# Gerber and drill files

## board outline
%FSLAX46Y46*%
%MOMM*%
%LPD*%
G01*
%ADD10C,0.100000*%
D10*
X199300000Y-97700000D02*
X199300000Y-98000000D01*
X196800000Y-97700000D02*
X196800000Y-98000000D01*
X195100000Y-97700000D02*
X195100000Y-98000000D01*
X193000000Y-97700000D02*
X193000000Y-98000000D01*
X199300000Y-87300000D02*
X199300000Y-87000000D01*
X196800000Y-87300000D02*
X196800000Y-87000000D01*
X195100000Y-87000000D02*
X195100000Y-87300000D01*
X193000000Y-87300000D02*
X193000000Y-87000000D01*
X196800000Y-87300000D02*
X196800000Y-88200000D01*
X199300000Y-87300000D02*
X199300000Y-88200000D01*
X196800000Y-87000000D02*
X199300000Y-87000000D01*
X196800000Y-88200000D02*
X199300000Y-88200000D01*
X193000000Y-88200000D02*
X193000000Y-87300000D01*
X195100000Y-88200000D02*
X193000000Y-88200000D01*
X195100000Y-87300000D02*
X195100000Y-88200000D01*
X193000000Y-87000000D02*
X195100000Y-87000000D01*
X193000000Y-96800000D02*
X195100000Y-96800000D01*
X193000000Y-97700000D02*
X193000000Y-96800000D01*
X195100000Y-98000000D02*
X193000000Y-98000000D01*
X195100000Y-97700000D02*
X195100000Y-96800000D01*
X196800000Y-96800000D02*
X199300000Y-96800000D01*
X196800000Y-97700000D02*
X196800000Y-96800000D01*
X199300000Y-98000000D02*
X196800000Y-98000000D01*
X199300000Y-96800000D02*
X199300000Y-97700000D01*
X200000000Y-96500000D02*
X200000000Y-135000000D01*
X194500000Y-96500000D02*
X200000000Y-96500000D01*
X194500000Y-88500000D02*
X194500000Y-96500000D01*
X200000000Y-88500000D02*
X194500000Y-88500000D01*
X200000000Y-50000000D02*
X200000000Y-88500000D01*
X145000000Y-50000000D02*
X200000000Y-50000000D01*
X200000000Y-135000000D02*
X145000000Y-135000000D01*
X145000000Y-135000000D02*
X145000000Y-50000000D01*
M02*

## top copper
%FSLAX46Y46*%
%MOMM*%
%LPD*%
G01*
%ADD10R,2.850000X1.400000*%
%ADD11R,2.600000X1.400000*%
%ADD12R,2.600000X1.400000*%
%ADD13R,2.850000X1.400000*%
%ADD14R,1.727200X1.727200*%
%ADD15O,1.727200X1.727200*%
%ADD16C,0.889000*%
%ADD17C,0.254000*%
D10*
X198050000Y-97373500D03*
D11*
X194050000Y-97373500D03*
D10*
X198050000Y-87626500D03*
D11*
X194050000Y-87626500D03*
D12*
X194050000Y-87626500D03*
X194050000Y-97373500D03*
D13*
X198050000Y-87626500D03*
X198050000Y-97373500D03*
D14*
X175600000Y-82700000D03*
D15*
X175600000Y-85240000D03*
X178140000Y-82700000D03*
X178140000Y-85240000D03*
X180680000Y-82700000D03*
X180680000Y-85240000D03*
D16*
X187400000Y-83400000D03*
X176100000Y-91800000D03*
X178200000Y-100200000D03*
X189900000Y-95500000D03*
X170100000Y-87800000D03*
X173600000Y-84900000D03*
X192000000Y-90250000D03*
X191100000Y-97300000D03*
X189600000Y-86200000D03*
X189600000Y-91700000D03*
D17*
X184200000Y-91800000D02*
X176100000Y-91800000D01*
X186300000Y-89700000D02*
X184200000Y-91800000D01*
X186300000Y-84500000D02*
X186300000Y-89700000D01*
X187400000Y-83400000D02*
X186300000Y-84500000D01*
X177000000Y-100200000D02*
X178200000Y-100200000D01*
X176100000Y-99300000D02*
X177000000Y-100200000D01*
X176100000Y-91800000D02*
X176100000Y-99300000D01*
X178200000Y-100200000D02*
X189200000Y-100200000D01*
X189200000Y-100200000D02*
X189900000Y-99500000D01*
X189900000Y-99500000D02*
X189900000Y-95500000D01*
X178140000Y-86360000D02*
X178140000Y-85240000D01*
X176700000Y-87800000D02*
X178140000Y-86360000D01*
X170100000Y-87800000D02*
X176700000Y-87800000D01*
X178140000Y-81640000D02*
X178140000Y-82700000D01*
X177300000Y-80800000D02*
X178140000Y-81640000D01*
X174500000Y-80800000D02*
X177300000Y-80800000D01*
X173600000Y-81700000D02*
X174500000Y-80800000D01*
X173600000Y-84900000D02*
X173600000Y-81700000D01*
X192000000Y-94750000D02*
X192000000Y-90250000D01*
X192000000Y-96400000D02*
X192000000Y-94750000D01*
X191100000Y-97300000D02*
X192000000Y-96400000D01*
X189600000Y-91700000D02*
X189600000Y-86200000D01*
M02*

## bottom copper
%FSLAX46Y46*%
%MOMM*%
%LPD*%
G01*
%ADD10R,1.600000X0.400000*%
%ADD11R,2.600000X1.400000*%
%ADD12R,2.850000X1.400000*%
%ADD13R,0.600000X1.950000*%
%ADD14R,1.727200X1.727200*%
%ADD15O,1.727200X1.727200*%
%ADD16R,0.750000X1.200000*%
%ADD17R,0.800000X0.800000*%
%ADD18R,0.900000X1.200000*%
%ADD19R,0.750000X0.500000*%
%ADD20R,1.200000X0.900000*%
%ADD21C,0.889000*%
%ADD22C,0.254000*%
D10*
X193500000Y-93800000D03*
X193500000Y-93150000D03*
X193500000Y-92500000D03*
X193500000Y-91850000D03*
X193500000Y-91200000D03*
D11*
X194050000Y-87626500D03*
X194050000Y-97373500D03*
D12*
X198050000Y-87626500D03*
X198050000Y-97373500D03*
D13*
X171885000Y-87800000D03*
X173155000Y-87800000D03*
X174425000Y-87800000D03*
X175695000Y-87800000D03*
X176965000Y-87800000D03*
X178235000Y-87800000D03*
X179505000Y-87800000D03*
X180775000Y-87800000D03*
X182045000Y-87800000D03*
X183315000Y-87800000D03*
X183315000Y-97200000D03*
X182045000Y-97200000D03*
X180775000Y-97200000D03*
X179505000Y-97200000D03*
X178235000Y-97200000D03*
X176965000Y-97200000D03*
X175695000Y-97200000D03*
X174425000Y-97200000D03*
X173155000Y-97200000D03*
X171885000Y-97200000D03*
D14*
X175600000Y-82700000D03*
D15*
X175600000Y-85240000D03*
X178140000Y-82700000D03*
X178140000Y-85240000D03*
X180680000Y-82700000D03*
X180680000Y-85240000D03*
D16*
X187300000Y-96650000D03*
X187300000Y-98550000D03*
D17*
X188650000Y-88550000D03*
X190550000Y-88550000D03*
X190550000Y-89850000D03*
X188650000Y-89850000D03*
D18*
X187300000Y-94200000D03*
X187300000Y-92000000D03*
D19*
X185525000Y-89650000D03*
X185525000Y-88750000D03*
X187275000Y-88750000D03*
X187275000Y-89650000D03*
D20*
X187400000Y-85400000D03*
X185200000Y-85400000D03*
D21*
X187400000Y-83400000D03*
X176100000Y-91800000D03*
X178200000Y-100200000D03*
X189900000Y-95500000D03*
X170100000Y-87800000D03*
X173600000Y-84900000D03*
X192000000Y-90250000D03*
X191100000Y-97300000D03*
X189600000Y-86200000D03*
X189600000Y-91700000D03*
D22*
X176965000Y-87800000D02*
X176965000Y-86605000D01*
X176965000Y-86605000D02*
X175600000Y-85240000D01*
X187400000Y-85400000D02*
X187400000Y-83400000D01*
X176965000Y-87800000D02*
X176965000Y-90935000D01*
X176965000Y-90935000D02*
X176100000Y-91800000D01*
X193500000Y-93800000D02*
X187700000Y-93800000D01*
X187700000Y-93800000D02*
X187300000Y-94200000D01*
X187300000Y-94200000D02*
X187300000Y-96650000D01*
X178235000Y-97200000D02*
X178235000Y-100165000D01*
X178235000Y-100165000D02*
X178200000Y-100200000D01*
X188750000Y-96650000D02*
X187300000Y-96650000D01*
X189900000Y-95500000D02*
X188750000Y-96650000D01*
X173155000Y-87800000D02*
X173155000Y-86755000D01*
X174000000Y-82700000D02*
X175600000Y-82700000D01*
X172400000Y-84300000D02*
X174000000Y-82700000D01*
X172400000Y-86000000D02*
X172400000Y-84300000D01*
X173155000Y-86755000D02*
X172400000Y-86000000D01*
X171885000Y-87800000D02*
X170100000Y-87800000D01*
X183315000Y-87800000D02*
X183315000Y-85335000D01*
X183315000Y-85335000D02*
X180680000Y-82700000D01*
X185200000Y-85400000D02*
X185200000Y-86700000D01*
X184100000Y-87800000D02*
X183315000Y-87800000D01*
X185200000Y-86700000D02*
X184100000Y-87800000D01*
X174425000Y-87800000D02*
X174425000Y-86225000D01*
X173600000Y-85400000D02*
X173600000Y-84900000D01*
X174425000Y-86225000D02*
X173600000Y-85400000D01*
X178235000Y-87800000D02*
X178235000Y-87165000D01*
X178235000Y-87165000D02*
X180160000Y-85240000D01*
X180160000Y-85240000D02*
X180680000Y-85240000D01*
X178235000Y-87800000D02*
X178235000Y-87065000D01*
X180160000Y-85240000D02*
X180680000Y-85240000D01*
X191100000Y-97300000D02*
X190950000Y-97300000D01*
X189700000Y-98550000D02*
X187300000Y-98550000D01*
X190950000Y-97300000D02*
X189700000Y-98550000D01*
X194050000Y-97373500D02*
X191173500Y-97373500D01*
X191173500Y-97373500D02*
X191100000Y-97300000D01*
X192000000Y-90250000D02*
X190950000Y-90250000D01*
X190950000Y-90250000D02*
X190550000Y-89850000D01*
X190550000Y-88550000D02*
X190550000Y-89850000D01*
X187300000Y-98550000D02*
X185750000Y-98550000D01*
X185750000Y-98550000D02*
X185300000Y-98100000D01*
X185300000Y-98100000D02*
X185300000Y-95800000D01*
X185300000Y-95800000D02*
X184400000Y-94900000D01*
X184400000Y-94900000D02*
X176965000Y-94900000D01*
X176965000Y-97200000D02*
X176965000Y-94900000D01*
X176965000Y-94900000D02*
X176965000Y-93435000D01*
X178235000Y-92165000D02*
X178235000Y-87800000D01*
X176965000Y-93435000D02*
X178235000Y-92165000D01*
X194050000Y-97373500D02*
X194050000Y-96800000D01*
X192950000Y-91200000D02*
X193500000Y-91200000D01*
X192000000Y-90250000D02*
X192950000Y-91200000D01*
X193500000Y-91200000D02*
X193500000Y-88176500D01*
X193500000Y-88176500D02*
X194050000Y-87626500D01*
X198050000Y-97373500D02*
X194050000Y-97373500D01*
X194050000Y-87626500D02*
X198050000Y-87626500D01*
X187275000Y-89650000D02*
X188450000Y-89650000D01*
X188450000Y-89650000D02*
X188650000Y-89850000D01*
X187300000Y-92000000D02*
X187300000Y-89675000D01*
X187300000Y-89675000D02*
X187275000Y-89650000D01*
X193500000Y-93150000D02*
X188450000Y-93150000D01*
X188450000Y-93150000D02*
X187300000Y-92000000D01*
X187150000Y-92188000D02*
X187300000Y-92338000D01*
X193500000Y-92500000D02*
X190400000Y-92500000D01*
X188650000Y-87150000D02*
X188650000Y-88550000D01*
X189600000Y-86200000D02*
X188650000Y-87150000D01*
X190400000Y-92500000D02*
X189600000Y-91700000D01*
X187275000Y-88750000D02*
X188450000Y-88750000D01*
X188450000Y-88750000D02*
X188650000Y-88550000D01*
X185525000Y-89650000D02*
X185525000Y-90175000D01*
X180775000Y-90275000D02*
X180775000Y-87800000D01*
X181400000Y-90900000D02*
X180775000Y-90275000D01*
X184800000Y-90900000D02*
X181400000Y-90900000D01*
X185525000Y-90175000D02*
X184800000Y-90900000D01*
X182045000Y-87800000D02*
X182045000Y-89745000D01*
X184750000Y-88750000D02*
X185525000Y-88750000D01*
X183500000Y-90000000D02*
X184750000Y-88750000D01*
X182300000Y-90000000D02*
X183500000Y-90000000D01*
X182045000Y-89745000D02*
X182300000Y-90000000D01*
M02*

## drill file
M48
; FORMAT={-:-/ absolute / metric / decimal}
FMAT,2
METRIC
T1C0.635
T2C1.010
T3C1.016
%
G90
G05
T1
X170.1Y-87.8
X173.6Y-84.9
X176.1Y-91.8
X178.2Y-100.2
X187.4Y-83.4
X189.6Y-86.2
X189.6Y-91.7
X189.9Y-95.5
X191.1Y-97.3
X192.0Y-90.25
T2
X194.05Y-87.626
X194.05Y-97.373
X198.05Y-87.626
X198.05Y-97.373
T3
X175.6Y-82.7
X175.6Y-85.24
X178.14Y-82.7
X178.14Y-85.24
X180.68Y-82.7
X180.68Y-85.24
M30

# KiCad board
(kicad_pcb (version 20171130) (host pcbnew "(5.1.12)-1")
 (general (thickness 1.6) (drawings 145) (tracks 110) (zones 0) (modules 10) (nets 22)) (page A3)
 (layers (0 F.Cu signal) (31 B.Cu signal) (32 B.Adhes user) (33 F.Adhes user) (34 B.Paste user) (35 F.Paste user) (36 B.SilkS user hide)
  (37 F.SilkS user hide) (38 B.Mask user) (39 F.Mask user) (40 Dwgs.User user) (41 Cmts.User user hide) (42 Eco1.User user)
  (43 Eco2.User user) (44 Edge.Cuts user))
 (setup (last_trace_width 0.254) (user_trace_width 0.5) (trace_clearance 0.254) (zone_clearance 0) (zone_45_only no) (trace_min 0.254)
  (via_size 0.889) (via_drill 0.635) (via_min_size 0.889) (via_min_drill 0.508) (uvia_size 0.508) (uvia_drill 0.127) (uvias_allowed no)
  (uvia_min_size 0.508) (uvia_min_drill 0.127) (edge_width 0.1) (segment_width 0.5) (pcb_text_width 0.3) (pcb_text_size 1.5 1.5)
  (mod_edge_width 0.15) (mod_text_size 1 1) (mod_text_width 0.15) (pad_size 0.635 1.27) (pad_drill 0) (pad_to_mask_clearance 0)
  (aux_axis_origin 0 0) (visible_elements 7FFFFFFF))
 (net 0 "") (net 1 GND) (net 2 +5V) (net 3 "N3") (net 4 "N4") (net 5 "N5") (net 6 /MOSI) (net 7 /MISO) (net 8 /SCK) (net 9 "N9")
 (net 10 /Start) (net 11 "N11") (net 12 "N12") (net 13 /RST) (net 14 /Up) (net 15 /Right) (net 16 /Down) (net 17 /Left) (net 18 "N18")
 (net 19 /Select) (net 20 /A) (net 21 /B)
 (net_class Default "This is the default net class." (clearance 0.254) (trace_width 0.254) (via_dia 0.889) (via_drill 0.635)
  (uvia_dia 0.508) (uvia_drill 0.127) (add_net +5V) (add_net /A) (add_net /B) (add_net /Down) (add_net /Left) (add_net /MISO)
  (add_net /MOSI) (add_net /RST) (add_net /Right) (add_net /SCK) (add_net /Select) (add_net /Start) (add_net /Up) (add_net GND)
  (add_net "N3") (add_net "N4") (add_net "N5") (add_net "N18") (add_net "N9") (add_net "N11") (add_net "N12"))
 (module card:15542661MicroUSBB (layer B.Cu) (at 194.5 92.5 270)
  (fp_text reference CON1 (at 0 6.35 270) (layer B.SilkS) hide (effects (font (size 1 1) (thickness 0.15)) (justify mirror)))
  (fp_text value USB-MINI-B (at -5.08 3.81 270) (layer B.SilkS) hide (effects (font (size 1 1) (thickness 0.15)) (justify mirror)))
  (pad 9 smd rect (at 4.8735 -3.55 270) (size 1.4 2.85) (layers F.Cu B.Paste B.Mask) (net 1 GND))
  (pad 7 smd rect (at 4.8735 0.45 270) (size 1.4 2.6) (layers F.Cu B.Paste B.Mask) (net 1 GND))
  (pad 8 smd rect (at -4.8735 -3.55 270) (size 1.4 2.85) (layers F.Cu B.Paste B.Mask) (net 1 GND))
  (pad 6 smd rect (at -4.8735 0.45 270) (size 1.4 2.6) (layers F.Cu B.Paste B.Mask) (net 1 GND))
  (pad 1 smd rect (at 1.3 1 270) (size 0.4 1.6) (layers B.Cu B.Paste B.Mask) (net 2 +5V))
  (pad 2 smd rect (at 0.65 1 270) (size 0.4 1.6) (layers B.Cu B.Paste B.Mask) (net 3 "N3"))
  (pad 3 smd rect (at 0 1 270) (size 0.4 1.6) (layers B.Cu B.Paste B.Mask) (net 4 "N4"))
  (pad 4 smd rect (at -0.65 1 270) (size 0.4 1.6) (layers B.Cu B.Paste B.Mask) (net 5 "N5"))
  (pad 5 smd rect (at -1.3 1 270) (size 0.4 1.6) (layers B.Cu B.Paste B.Mask) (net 1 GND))
  (pad 6 thru_hole rect (at -4.8735 0.45 270) (size 1.4 2.6) (drill 1.01) (layers *.Cu *.Mask B.SilkS) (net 1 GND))
  (pad 7 thru_hole rect (at 4.8735 0.45 270) (size 1.4 2.6) (drill 1.01) (layers *.Cu *.Mask B.SilkS) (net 1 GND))
  (pad 8 thru_hole rect (at -4.8735 -3.55 270) (size 1.4 2.85) (drill 1.01) (layers *.Cu *.Mask B.SilkS) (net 1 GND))
  (pad 9 thru_hole rect (at 4.8735 -3.55 270) (size 1.4 2.85) (drill 1.01) (layers *.Cu *.Mask B.SilkS) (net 1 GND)))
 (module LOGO (layer F.Cu) (at 152.75 72 270)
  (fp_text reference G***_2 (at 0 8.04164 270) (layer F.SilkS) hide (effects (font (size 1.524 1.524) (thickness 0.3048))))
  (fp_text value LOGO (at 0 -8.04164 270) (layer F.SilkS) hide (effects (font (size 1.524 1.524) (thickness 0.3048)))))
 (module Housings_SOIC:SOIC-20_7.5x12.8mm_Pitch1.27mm (layer B.Cu) (at 177.6 92.5 270)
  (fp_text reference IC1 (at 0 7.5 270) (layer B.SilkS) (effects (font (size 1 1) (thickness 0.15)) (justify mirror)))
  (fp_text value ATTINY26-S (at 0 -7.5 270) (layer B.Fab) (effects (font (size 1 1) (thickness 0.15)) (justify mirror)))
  (pad 1 smd rect (at -4.7 5.715 270) (size 1.95 0.6) (layers B.Cu B.Paste B.Mask) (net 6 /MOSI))
  (pad 2 smd rect (at -4.7 4.445 270) (size 1.95 0.6) (layers B.Cu B.Paste B.Mask) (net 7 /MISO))
  (pad 3 smd rect (at -4.7 3.175 270) (size 1.95 0.6) (layers B.Cu B.Paste B.Mask) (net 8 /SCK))
  (pad 4 smd rect (at -4.7 1.905 270) (size 1.95 0.6) (layers B.Cu B.Paste B.Mask) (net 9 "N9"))
  (pad 5 smd rect (at -4.7 0.635 270) (size 1.95 0.6) (layers B.Cu B.Paste B.Mask) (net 2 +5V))
  (pad 6 smd rect (at -4.7 -0.635 270) (size 1.95 0.6) (layers B.Cu B.Paste B.Mask) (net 1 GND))
  (pad 7 smd rect (at -4.7 -1.905 270) (size 1.95 0.6) (layers B.Cu B.Paste B.Mask) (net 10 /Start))
  (pad 8 smd rect (at -4.7 -3.175 270) (size 1.95 0.6) (layers B.Cu B.Paste B.Mask) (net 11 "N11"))
  (pad 9 smd rect (at -4.7 -4.445 270) (size 1.95 0.6) (layers B.Cu B.Paste B.Mask) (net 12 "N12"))
  (pad 10 smd rect (at -4.7 -5.715 270) (size 1.95 0.6) (layers B.Cu B.Paste B.Mask) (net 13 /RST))
  (pad 11 smd rect (at 4.7 -5.715 270) (size 1.95 0.6) (layers B.Cu B.Paste B.Mask) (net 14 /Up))
  (pad 12 smd rect (at 4.7 -4.445 270) (size 1.95 0.6) (layers B.Cu B.Paste B.Mask) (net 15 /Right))
  (pad 13 smd rect (at 4.7 -3.175 270) (size 1.95 0.6) (layers B.Cu B.Paste B.Mask) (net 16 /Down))
  (pad 14 smd rect (at 4.7 -1.905 270) (size 1.95 0.6) (layers B.Cu B.Paste B.Mask) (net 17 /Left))
  (pad 15 smd rect (at 4.7 -0.635 270) (size 1.95 0.6) (layers B.Cu B.Paste B.Mask) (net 2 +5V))
  (pad 16 smd rect (at 4.7 0.635 270) (size 1.95 0.6) (layers B.Cu B.Paste B.Mask) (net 1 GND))
  (pad 17 smd rect (at 4.7 1.905 270) (size 1.95 0.6) (layers B.Cu B.Paste B.Mask) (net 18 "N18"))
  (pad 18 smd rect (at 4.7 3.175 270) (size 1.95 0.6) (layers B.Cu B.Paste B.Mask) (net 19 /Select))
  (pad 19 smd rect (at 4.7 4.445 270) (size 1.95 0.6) (layers B.Cu B.Paste B.Mask) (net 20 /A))
  (pad 20 smd rect (at 4.7 5.715 270) (size 1.95 0.6) (layers B.Cu B.Paste B.Mask) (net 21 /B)))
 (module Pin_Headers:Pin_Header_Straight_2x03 (layer B.Cu) (at 175.6 82.7 270)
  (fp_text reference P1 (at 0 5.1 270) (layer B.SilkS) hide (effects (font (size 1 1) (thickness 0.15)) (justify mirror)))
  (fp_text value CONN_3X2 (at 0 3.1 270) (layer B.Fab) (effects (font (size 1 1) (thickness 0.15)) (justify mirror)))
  (pad 1 thru_hole rect (at 0 0 270) (size 1.7272 1.7272) (drill 1.016) (layers *.Cu *.Mask B.SilkS) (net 7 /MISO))
  (pad 2 thru_hole oval (at 2.54 0 270) (size 1.7272 1.7272) (drill 1.016) (layers *.Cu *.Mask B.SilkS) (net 2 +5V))
  (pad 3 thru_hole oval (at 0 -2.54 270) (size 1.7272 1.7272) (drill 1.016) (layers *.Cu *.Mask B.SilkS) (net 8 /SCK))
  (pad 4 thru_hole oval (at 2.54 -2.54 270) (size 1.7272 1.7272) (drill 1.016) (layers *.Cu *.Mask B.SilkS) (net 6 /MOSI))
  (pad 5 thru_hole oval (at 0 -5.08 270) (size 1.7272 1.7272) (drill 1.016) (layers *.Cu *.Mask B.SilkS) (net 13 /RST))
  (pad 6 thru_hole oval (at 2.54 -5.08 270) (size 1.7272 1.7272) (drill 1.016) (layers *.Cu *.Mask B.SilkS) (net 1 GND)))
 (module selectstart (layer B.Cu) (at 168.5 92.5 270)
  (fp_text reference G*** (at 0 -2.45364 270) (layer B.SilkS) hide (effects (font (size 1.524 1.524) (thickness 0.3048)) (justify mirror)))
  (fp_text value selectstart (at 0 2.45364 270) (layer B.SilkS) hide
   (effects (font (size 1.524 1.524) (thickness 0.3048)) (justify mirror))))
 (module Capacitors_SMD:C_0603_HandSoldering (layer B.Cu) (at 187.3 97.6 270)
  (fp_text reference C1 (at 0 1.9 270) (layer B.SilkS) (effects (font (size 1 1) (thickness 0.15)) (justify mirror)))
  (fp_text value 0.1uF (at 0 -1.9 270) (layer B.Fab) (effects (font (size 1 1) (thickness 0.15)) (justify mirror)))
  (pad 1 smd rect (at -0.95 0 270) (size 1.2 0.75) (layers B.Cu B.Paste B.Mask) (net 2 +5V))
  (pad 2 smd rect (at 0.95 0 270) (size 1.2 0.75) (layers B.Cu B.Paste B.Mask) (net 1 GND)))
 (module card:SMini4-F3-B (layer B.Cu) (at 189.6 89.2 270)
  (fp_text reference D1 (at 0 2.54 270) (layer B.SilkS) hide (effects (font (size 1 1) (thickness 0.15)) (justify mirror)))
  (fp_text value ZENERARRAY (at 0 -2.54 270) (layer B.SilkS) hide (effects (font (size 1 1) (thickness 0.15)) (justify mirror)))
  (pad 4 smd rect (at -0.65 0.95 270) (size 0.8 0.8) (layers B.Cu B.Paste B.Mask) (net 4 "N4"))
  (pad 1 smd rect (at -0.65 -0.95 270) (size 0.8 0.8) (layers B.Cu B.Paste B.Mask) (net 1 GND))
  (pad 2 smd rect (at 0.65 -0.95 270) (size 0.8 0.8) (layers B.Cu B.Paste B.Mask) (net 1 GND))
  (pad 3 smd rect (at 0.65 0.95 270) (size 0.8 0.8) (layers B.Cu B.Paste B.Mask) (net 3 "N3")))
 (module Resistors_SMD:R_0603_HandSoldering (layer B.Cu) (at 187.3 93.1 90)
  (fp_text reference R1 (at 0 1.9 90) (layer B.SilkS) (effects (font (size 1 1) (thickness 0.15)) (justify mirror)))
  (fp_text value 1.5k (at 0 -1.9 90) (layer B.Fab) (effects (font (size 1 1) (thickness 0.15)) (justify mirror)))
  (pad 1 smd rect (at -1.1 0 90) (size 1.2 0.9) (layers B.Cu B.Paste B.Mask) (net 2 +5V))
  (pad 2 smd rect (at 1.1 0 90) (size 1.2 0.9) (layers B.Cu B.Paste B.Mask) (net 3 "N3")))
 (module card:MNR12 (layer B.Cu) (at 186.4 89.2 90)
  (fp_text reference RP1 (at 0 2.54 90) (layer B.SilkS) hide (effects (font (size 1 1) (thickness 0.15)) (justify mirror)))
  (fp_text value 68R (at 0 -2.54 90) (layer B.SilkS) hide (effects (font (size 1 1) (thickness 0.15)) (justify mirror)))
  (pad 1 smd rect (at -0.45 -0.875 90) (size 0.5 0.75) (layers B.Cu B.Paste B.Mask) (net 11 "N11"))
  (pad 2 smd rect (at 0.45 -0.875 90) (size 0.5 0.75) (layers B.Cu B.Paste B.Mask) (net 12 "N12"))
  (pad 3 smd rect (at 0.45 0.875 90) (size 0.5 0.75) (layers B.Cu B.Paste B.Mask) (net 4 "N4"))
  (pad 4 smd rect (at -0.45 0.875 90) (size 0.5 0.75) (layers B.Cu B.Paste B.Mask) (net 3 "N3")))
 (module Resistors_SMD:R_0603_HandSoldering (layer B.Cu) (at 186.3 85.4 180)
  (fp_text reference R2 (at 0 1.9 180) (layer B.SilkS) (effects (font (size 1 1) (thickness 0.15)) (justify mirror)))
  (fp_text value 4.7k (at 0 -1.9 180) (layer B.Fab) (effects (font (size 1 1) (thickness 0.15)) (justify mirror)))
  (pad 1 smd rect (at -1.1 0 180) (size 1.2 0.9) (layers B.Cu B.Paste B.Mask) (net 2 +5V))
  (pad 2 smd rect (at 1.1 0 180) (size 1.2 0.9) (layers B.Cu B.Paste B.Mask) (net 13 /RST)))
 (gr_line (start 199.3 97.7) (end 199.3 98) (angle 90) (layer Edge.Cuts) (width 0.1))
 (gr_line (start 196.8 97.7) (end 196.8 98) (angle 90) (layer Edge.Cuts) (width 0.1))
 (gr_line (start 195.1 97.7) (end 195.1 98) (angle 90) (layer Edge.Cuts) (width 0.1))
 (gr_line (start 193 97.7) (end 193 98) (angle 90) (layer Edge.Cuts) (width 0.1))
 (gr_line (start 199.3 87.3) (end 199.3 87) (angle 90) (layer Edge.Cuts) (width 0.1))
 (gr_line (start 196.8 87.3) (end 196.8 87) (angle 90) (layer Edge.Cuts) (width 0.1))
 (gr_line (start 195.1 87) (end 195.1 87.3) (angle 90) (layer Edge.Cuts) (width 0.1))
 (gr_line (start 193 87.3) (end 193 87) (angle 90) (layer Edge.Cuts) (width 0.1))
 (gr_line (start 196.8 87.3) (end 196.8 88.2) (angle 90) (layer Edge.Cuts) (width 0.1))
 (gr_line (start 199.3 87.3) (end 199.3 88.2) (angle 90) (layer Edge.Cuts) (width 0.1))
 (gr_line (start 196.8 87) (end 199.3 87) (angle 90) (layer Edge.Cuts) (width 0.1))
 (gr_line (start 196.8 88.2) (end 199.3 88.2) (angle 90) (layer Edge.Cuts) (width 0.1))
 (gr_line (start 193 88.2) (end 193 87.3) (angle 90) (layer Edge.Cuts) (width 0.1))
 (gr_line (start 195.1 88.2) (end 193 88.2) (angle 90) (layer Edge.Cuts) (width 0.1))
 (gr_line (start 195.1 87.3) (end 195.1 88.2) (angle 90) (layer Edge.Cuts) (width 0.1))
 (gr_line (start 193 87) (end 195.1 87) (angle 90) (layer Edge.Cuts) (width 0.1))
 (gr_line (start 193 96.8) (end 195.1 96.8) (angle 90) (layer Edge.Cuts) (width 0.1))
 (gr_line (start 193 97.7) (end 193 96.8) (angle 90) (layer Edge.Cuts) (width 0.1))
 (gr_line (start 195.1 98) (end 193 98) (angle 90) (layer Edge.Cuts) (width 0.1))
 (gr_line (start 195.1 97.7) (end 195.1 96.8) (angle 90) (layer Edge.Cuts) (width 0.1))
 (gr_line (start 196.8 96.8) (end 199.3 96.8) (angle 90) (layer Edge.Cuts) (width 0.1))
 (gr_line (start 196.8 97.7) (end 196.8 96.8) (angle 90) (layer Edge.Cuts) (width 0.1))
 (gr_line (start 199.3 98) (end 196.8 98) (angle 90) (layer Edge.Cuts) (width 0.1))
 (gr_line (start 199.3 96.8) (end 199.3 97.7) (angle 90) (layer Edge.Cuts) (width 0.1))
 (gr_line (start 200 96.5) (end 200 135) (angle 90) (layer Edge.Cuts) (width 0.1))
 (gr_line (start 194.5 96.5) (end 200 96.5) (angle 90) (layer Edge.Cuts) (width 0.1))
 (gr_line (start 194.5 88.5) (end 194.5 96.5) (angle 90) (layer Edge.Cuts) (width 0.1))
 (gr_line (start 200 88.5) (end 194.5 88.5) (angle 90) (layer Edge.Cuts) (width 0.1))
 (gr_line (start 200 50) (end 200 88.5) (angle 90) (layer Edge.Cuts) (width 0.1))
 (gr_line (start 145 50) (end 200 50) (angle 90) (layer Edge.Cuts) (width 0.1))
 (gr_line (start 200 135) (end 145 135) (angle 90) (layer Edge.Cuts) (width 0.1))
 (gr_line (start 145 135) (end 145 50) (angle 90) (layer Edge.Cuts) (width 0.1))
 (segment (start 176.965 87.8) (end 176.965 86.605) (width 0.254) (layer B.Cu) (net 2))
 (segment (start 176.965 86.605) (end 175.6 85.24) (width 0.254) (layer B.Cu) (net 2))
 (segment (start 187.4 85.4) (end 187.4 83.4) (width 0.254) (layer B.Cu) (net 2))
 (segment (start 184.2 91.8) (end 176.1 91.8) (width 0.254) (layer F.Cu) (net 2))
 (segment (start 186.3 89.7) (end 184.2 91.8) (width 0.254) (layer F.Cu) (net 2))
 (segment (start 186.3 84.5) (end 186.3 89.7) (width 0.254) (layer F.Cu) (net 2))
 (segment (start 187.4 83.4) (end 186.3 84.5) (width 0.254) (layer F.Cu) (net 2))
 (segment (start 176.965 87.8) (end 176.965 90.935) (width 0.254) (layer B.Cu) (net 2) (status 10))
 (segment (start 177 100.2) (end 178.2 100.2) (width 0.254) (layer F.Cu) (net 2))
 (segment (start 176.1 99.3) (end 177 100.2) (width 0.254) (layer F.Cu) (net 2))
 (segment (start 176.1 91.8) (end 176.1 99.3) (width 0.254) (layer F.Cu) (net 2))
 (segment (start 176.965 90.935) (end 176.1 91.8) (width 0.254) (layer B.Cu) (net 2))
 (segment (start 193.5 93.8) (end 187.7 93.8) (width 0.254) (layer B.Cu) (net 2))
 (segment (start 187.7 93.8) (end 187.3 94.2) (width 0.254) (layer B.Cu) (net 2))
 (segment (start 187.3 94.2) (end 187.3 96.65) (width 0.254) (layer B.Cu) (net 2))
 (segment (start 178.235 97.2) (end 178.235 100.165) (width 0.254) (layer B.Cu) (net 2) (status 10))
 (segment (start 178.235 100.165) (end 178.2 100.2) (width 0.254) (layer B.Cu) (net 2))
 (segment (start 188.75 96.65) (end 187.3 96.65) (width 0.254) (layer B.Cu) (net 2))
 (segment (start 178.2 100.2) (end 189.2 100.2) (width 0.254) (layer F.Cu) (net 2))
 (segment (start 189.2 100.2) (end 189.9 99.5) (width 0.254) (layer F.Cu) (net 2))
 (segment (start 189.9 99.5) (end 189.9 95.5) (width 0.254) (layer F.Cu) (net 2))
 (segment (start 189.9 95.5) (end 188.75 96.65) (width 0.254) (layer B.Cu) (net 2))
 (via (at 187.4 83.4) (size 0.889) (drill 0.635) (layers F.Cu B.Cu) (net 2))
 (via (at 176.1 91.8) (size 0.889) (drill 0.635) (layers F.Cu B.Cu) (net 2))
 (via (at 178.2 100.2) (size 0.889) (drill 0.635) (layers F.Cu B.Cu) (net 2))
 (via (at 189.9 95.5) (size 0.889) (drill 0.635) (layers F.Cu B.Cu) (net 2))
 (segment (start 173.155 87.8) (end 173.155 86.755) (width 0.254) (layer B.Cu) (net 7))
 (segment (start 174 82.7) (end 175.6 82.7) (width 0.254) (layer B.Cu) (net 7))
 (segment (start 172.4 84.3) (end 174 82.7) (width 0.254) (layer B.Cu) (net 7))
 (segment (start 172.4 86) (end 172.4 84.3) (width 0.254) (layer B.Cu) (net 7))
 (segment (start 173.155 86.755) (end 172.4 86) (width 0.254) (layer B.Cu) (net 7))
 (segment (start 171.885 87.8) (end 170.1 87.8) (width 0.254) (layer B.Cu) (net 6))
 (segment (start 178.14 86.36) (end 178.14 85.24) (width 0.254) (layer F.Cu) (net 6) (status 20))
 (segment (start 176.7 87.8) (end 178.14 86.36) (width 0.254) (layer F.Cu) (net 6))
 (segment (start 170.1 87.8) (end 176.7 87.8) (width 0.254) (layer F.Cu) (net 6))
 (via (at 170.1 87.8) (size 0.889) (drill 0.635) (layers F.Cu B.Cu) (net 6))
 (segment (start 183.315 87.8) (end 183.315 85.335) (width 0.254) (layer B.Cu) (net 13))
 (segment (start 183.315 85.335) (end 180.68 82.7) (width 0.254) (layer B.Cu) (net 13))
 (segment (start 185.2 85.4) (end 185.2 86.7) (width 0.254) (layer B.Cu) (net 13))
 (segment (start 184.1 87.8) (end 183.315 87.8) (width 0.254) (layer B.Cu) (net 13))
 (segment (start 185.2 86.7) (end 184.1 87.8) (width 0.254) (layer B.Cu) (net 13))
 (segment (start 174.425 87.8) (end 174.425 86.225) (width 0.254) (layer B.Cu) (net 8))
 (segment (start 178.14 81.64) (end 178.14 82.7) (width 0.254) (layer F.Cu) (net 8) (status 20))
 (segment (start 177.3 80.8) (end 178.14 81.64) (width 0.254) (layer F.Cu) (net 8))
 (segment (start 174.5 80.8) (end 177.3 80.8) (width 0.254) (layer F.Cu) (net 8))
 (segment (start 173.6 81.7) (end 174.5 80.8) (width 0.254) (layer F.Cu) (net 8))
 (segment (start 173.6 84.9) (end 173.6 81.7) (width 0.254) (layer F.Cu) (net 8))
 (segment (start 173.6 85.4) (end 173.6 84.9) (width 0.254) (layer B.Cu) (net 8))
 (segment (start 174.425 86.225) (end 173.6 85.4) (width 0.254) (layer B.Cu) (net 8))
 (via (at 173.6 84.9) (size 0.889) (drill 0.635) (layers F.Cu B.Cu) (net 8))
 (segment (start 178.235 87.8) (end 178.235 87.165) (width 0.254) (layer B.Cu) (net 1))
 (segment (start 178.235 87.165) (end 180.16 85.24) (width 0.254) (layer B.Cu) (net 1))
 (segment (start 180.16 85.24) (end 180.68 85.24) (width 0.254) (layer B.Cu) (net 1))
 (segment (start 178.235 87.8) (end 178.235 87.065) (width 0.254) (layer B.Cu) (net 1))
 (segment (start 180.16 85.24) (end 180.68 85.24) (width 0.254) (layer B.Cu) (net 1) (status 30))
 (segment (start 191.1 97.3) (end 190.95 97.3) (width 0.254) (layer B.Cu) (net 1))
 (segment (start 189.7 98.55) (end 187.3 98.55) (width 0.254) (layer B.Cu) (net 1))
 (segment (start 190.95 97.3) (end 189.7 98.55) (width 0.254) (layer B.Cu) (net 1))
 (segment (start 194.05 97.3735) (end 191.1735 97.3735) (width 0.254) (layer B.Cu) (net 1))
 (segment (start 192 94.75) (end 192 90.25) (width 0.254) (layer F.Cu) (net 1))
 (segment (start 192 96.4) (end 192 94.75) (width 0.254) (layer F.Cu) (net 1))
 (segment (start 191.1 97.3) (end 192 96.4) (width 0.254) (layer F.Cu) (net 1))
 (segment (start 191.1735 97.3735) (end 191.1 97.3) (width 0.254) (layer B.Cu) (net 1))
 (segment (start 192 90.25) (end 190.95 90.25) (width 0.254) (layer B.Cu) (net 1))
 (segment (start 190.95 90.25) (end 190.55 89.85) (width 0.254) (layer B.Cu) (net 1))
 (segment (start 190.55 88.55) (end 190.55 89.85) (width 0.254) (layer B.Cu) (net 1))
 (segment (start 187.3 98.55) (end 185.75 98.55) (width 0.254) (layer B.Cu) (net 1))
 (segment (start 185.75 98.55) (end 185.3 98.1) (width 0.254) (layer B.Cu) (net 1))
 (segment (start 185.3 98.1) (end 185.3 95.8) (width 0.254) (layer B.Cu) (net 1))
 (segment (start 185.3 95.8) (end 184.4 94.9) (width 0.254) (layer B.Cu) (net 1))
 (segment (start 184.4 94.9) (end 176.965 94.9) (width 0.254) (layer B.Cu) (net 1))
 (segment (start 176.965 97.2) (end 176.965 94.9) (width 0.254) (layer B.Cu) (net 1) (status 10))
 (segment (start 176.965 94.9) (end 176.965 93.435) (width 0.254) (layer B.Cu) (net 1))
 (segment (start 178.235 92.165) (end 178.235 87.8) (width 0.254) (layer B.Cu) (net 1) (status 20))
 (segment (start 176.965 93.435) (end 178.235 92.165) (width 0.254) (layer B.Cu) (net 1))
 (segment (start 194.05 97.3735) (end 194.05 96.8) (width 0.254) (layer B.Cu) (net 1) (status 30))
 (segment (start 192.95 91.2) (end 193.5 91.2) (width 0.254) (layer B.Cu) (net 1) (status 30))
 (segment (start 192 90.25) (end 192.95 91.2) (width 0.254) (layer B.Cu) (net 1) (status 20))
 (segment (start 193.5 91.2) (end 193.5 88.1765) (width 0.254) (layer B.Cu) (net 1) (status 30))
 (segment (start 193.5 88.1765) (end 194.05 87.6265) (width 0.254) (layer B.Cu) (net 1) (status 30))
 (segment (start 198.05 97.3735) (end 194.05 97.3735) (width 0.254) (layer B.Cu) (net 1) (status 30))
 (segment (start 194.05 87.6265) (end 198.05 87.6265) (width 0.254) (layer B.Cu) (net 1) (status 30))
 (via (at 192 90.25) (size 0.889) (layers F.Cu B.Cu) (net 1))
 (via (at 191.1 97.3) (size 0.889) (drill 0.635) (layers F.Cu B.Cu) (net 1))
 (segment (start 187.275 89.65) (end 188.45 89.65) (width 0.254) (layer B.Cu) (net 3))
 (segment (start 188.45 89.65) (end 188.65 89.85) (width 0.254) (layer B.Cu) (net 3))
 (segment (start 187.3 92) (end 187.3 89.675) (width 0.254) (layer B.Cu) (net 3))
 (segment (start 187.3 89.675) (end 187.275 89.65) (width 0.254) (layer B.Cu) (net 3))
 (segment (start 193.5 93.15) (end 188.45 93.15) (width 0.254) (layer B.Cu) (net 3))
 (segment (start 188.45 93.15) (end 187.3 92) (width 0.254) (layer B.Cu) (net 3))
 (segment (start 187.15 92.188) (end 187.3 92.338) (width 0.254) (layer B.Cu) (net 3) (status 30))
 (segment (start 193.5 92.5) (end 190.4 92.5) (width 0.254) (layer B.Cu) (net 4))
 (segment (start 188.65 87.15) (end 188.65 88.55) (width 0.254) (layer B.Cu) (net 4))
 (segment (start 189.6 86.2) (end 188.65 87.15) (width 0.254) (layer B.Cu) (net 4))
 (segment (start 189.6 91.7) (end 189.6 86.2) (width 0.254) (layer F.Cu) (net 4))
 (segment (start 190.4 92.5) (end 189.6 91.7) (width 0.254) (layer B.Cu) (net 4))
 (segment (start 187.275 88.75) (end 188.45 88.75) (width 0.254) (layer B.Cu) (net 4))
 (segment (start 188.45 88.75) (end 188.65 88.55) (width 0.254) (layer B.Cu) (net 4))
 (via (at 189.6 86.2) (size 0.889) (drill 0.635) (layers F.Cu B.Cu) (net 4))
 (via (at 189.6 91.7) (size 0.889) (drill 0.635) (layers F.Cu B.Cu) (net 4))
 (segment (start 185.525 89.65) (end 185.525 90.175) (width 0.254) (layer B.Cu) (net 11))
 (segment (start 180.775 90.275) (end 180.775 87.8) (width 0.254) (layer B.Cu) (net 11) (status 20))
 (segment (start 181.4 90.9) (end 180.775 90.275) (width 0.254) (layer B.Cu) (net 11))
 (segment (start 184.8 90.9) (end 181.4 90.9) (width 0.254) (layer B.Cu) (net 11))
 (segment (start 185.525 90.175) (end 184.8 90.9) (width 0.254) (layer B.Cu) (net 11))
 (segment (start 182.045 87.8) (end 182.045 89.745) (width 0.254) (layer B.Cu) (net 12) (status 10))
 (segment (start 184.75 88.75) (end 185.525 88.75) (width 0.254) (layer B.Cu) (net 12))
 (segment (start 183.5 90) (end 184.75 88.75) (width 0.254) (layer B.Cu) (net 12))
 (segment (start 182.3 90) (end 183.5 90) (width 0.254) (layer B.Cu) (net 12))
 (segment (start 182.045 89.745) (end 182.3 90) (width 0.254) (layer B.Cu) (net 12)))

